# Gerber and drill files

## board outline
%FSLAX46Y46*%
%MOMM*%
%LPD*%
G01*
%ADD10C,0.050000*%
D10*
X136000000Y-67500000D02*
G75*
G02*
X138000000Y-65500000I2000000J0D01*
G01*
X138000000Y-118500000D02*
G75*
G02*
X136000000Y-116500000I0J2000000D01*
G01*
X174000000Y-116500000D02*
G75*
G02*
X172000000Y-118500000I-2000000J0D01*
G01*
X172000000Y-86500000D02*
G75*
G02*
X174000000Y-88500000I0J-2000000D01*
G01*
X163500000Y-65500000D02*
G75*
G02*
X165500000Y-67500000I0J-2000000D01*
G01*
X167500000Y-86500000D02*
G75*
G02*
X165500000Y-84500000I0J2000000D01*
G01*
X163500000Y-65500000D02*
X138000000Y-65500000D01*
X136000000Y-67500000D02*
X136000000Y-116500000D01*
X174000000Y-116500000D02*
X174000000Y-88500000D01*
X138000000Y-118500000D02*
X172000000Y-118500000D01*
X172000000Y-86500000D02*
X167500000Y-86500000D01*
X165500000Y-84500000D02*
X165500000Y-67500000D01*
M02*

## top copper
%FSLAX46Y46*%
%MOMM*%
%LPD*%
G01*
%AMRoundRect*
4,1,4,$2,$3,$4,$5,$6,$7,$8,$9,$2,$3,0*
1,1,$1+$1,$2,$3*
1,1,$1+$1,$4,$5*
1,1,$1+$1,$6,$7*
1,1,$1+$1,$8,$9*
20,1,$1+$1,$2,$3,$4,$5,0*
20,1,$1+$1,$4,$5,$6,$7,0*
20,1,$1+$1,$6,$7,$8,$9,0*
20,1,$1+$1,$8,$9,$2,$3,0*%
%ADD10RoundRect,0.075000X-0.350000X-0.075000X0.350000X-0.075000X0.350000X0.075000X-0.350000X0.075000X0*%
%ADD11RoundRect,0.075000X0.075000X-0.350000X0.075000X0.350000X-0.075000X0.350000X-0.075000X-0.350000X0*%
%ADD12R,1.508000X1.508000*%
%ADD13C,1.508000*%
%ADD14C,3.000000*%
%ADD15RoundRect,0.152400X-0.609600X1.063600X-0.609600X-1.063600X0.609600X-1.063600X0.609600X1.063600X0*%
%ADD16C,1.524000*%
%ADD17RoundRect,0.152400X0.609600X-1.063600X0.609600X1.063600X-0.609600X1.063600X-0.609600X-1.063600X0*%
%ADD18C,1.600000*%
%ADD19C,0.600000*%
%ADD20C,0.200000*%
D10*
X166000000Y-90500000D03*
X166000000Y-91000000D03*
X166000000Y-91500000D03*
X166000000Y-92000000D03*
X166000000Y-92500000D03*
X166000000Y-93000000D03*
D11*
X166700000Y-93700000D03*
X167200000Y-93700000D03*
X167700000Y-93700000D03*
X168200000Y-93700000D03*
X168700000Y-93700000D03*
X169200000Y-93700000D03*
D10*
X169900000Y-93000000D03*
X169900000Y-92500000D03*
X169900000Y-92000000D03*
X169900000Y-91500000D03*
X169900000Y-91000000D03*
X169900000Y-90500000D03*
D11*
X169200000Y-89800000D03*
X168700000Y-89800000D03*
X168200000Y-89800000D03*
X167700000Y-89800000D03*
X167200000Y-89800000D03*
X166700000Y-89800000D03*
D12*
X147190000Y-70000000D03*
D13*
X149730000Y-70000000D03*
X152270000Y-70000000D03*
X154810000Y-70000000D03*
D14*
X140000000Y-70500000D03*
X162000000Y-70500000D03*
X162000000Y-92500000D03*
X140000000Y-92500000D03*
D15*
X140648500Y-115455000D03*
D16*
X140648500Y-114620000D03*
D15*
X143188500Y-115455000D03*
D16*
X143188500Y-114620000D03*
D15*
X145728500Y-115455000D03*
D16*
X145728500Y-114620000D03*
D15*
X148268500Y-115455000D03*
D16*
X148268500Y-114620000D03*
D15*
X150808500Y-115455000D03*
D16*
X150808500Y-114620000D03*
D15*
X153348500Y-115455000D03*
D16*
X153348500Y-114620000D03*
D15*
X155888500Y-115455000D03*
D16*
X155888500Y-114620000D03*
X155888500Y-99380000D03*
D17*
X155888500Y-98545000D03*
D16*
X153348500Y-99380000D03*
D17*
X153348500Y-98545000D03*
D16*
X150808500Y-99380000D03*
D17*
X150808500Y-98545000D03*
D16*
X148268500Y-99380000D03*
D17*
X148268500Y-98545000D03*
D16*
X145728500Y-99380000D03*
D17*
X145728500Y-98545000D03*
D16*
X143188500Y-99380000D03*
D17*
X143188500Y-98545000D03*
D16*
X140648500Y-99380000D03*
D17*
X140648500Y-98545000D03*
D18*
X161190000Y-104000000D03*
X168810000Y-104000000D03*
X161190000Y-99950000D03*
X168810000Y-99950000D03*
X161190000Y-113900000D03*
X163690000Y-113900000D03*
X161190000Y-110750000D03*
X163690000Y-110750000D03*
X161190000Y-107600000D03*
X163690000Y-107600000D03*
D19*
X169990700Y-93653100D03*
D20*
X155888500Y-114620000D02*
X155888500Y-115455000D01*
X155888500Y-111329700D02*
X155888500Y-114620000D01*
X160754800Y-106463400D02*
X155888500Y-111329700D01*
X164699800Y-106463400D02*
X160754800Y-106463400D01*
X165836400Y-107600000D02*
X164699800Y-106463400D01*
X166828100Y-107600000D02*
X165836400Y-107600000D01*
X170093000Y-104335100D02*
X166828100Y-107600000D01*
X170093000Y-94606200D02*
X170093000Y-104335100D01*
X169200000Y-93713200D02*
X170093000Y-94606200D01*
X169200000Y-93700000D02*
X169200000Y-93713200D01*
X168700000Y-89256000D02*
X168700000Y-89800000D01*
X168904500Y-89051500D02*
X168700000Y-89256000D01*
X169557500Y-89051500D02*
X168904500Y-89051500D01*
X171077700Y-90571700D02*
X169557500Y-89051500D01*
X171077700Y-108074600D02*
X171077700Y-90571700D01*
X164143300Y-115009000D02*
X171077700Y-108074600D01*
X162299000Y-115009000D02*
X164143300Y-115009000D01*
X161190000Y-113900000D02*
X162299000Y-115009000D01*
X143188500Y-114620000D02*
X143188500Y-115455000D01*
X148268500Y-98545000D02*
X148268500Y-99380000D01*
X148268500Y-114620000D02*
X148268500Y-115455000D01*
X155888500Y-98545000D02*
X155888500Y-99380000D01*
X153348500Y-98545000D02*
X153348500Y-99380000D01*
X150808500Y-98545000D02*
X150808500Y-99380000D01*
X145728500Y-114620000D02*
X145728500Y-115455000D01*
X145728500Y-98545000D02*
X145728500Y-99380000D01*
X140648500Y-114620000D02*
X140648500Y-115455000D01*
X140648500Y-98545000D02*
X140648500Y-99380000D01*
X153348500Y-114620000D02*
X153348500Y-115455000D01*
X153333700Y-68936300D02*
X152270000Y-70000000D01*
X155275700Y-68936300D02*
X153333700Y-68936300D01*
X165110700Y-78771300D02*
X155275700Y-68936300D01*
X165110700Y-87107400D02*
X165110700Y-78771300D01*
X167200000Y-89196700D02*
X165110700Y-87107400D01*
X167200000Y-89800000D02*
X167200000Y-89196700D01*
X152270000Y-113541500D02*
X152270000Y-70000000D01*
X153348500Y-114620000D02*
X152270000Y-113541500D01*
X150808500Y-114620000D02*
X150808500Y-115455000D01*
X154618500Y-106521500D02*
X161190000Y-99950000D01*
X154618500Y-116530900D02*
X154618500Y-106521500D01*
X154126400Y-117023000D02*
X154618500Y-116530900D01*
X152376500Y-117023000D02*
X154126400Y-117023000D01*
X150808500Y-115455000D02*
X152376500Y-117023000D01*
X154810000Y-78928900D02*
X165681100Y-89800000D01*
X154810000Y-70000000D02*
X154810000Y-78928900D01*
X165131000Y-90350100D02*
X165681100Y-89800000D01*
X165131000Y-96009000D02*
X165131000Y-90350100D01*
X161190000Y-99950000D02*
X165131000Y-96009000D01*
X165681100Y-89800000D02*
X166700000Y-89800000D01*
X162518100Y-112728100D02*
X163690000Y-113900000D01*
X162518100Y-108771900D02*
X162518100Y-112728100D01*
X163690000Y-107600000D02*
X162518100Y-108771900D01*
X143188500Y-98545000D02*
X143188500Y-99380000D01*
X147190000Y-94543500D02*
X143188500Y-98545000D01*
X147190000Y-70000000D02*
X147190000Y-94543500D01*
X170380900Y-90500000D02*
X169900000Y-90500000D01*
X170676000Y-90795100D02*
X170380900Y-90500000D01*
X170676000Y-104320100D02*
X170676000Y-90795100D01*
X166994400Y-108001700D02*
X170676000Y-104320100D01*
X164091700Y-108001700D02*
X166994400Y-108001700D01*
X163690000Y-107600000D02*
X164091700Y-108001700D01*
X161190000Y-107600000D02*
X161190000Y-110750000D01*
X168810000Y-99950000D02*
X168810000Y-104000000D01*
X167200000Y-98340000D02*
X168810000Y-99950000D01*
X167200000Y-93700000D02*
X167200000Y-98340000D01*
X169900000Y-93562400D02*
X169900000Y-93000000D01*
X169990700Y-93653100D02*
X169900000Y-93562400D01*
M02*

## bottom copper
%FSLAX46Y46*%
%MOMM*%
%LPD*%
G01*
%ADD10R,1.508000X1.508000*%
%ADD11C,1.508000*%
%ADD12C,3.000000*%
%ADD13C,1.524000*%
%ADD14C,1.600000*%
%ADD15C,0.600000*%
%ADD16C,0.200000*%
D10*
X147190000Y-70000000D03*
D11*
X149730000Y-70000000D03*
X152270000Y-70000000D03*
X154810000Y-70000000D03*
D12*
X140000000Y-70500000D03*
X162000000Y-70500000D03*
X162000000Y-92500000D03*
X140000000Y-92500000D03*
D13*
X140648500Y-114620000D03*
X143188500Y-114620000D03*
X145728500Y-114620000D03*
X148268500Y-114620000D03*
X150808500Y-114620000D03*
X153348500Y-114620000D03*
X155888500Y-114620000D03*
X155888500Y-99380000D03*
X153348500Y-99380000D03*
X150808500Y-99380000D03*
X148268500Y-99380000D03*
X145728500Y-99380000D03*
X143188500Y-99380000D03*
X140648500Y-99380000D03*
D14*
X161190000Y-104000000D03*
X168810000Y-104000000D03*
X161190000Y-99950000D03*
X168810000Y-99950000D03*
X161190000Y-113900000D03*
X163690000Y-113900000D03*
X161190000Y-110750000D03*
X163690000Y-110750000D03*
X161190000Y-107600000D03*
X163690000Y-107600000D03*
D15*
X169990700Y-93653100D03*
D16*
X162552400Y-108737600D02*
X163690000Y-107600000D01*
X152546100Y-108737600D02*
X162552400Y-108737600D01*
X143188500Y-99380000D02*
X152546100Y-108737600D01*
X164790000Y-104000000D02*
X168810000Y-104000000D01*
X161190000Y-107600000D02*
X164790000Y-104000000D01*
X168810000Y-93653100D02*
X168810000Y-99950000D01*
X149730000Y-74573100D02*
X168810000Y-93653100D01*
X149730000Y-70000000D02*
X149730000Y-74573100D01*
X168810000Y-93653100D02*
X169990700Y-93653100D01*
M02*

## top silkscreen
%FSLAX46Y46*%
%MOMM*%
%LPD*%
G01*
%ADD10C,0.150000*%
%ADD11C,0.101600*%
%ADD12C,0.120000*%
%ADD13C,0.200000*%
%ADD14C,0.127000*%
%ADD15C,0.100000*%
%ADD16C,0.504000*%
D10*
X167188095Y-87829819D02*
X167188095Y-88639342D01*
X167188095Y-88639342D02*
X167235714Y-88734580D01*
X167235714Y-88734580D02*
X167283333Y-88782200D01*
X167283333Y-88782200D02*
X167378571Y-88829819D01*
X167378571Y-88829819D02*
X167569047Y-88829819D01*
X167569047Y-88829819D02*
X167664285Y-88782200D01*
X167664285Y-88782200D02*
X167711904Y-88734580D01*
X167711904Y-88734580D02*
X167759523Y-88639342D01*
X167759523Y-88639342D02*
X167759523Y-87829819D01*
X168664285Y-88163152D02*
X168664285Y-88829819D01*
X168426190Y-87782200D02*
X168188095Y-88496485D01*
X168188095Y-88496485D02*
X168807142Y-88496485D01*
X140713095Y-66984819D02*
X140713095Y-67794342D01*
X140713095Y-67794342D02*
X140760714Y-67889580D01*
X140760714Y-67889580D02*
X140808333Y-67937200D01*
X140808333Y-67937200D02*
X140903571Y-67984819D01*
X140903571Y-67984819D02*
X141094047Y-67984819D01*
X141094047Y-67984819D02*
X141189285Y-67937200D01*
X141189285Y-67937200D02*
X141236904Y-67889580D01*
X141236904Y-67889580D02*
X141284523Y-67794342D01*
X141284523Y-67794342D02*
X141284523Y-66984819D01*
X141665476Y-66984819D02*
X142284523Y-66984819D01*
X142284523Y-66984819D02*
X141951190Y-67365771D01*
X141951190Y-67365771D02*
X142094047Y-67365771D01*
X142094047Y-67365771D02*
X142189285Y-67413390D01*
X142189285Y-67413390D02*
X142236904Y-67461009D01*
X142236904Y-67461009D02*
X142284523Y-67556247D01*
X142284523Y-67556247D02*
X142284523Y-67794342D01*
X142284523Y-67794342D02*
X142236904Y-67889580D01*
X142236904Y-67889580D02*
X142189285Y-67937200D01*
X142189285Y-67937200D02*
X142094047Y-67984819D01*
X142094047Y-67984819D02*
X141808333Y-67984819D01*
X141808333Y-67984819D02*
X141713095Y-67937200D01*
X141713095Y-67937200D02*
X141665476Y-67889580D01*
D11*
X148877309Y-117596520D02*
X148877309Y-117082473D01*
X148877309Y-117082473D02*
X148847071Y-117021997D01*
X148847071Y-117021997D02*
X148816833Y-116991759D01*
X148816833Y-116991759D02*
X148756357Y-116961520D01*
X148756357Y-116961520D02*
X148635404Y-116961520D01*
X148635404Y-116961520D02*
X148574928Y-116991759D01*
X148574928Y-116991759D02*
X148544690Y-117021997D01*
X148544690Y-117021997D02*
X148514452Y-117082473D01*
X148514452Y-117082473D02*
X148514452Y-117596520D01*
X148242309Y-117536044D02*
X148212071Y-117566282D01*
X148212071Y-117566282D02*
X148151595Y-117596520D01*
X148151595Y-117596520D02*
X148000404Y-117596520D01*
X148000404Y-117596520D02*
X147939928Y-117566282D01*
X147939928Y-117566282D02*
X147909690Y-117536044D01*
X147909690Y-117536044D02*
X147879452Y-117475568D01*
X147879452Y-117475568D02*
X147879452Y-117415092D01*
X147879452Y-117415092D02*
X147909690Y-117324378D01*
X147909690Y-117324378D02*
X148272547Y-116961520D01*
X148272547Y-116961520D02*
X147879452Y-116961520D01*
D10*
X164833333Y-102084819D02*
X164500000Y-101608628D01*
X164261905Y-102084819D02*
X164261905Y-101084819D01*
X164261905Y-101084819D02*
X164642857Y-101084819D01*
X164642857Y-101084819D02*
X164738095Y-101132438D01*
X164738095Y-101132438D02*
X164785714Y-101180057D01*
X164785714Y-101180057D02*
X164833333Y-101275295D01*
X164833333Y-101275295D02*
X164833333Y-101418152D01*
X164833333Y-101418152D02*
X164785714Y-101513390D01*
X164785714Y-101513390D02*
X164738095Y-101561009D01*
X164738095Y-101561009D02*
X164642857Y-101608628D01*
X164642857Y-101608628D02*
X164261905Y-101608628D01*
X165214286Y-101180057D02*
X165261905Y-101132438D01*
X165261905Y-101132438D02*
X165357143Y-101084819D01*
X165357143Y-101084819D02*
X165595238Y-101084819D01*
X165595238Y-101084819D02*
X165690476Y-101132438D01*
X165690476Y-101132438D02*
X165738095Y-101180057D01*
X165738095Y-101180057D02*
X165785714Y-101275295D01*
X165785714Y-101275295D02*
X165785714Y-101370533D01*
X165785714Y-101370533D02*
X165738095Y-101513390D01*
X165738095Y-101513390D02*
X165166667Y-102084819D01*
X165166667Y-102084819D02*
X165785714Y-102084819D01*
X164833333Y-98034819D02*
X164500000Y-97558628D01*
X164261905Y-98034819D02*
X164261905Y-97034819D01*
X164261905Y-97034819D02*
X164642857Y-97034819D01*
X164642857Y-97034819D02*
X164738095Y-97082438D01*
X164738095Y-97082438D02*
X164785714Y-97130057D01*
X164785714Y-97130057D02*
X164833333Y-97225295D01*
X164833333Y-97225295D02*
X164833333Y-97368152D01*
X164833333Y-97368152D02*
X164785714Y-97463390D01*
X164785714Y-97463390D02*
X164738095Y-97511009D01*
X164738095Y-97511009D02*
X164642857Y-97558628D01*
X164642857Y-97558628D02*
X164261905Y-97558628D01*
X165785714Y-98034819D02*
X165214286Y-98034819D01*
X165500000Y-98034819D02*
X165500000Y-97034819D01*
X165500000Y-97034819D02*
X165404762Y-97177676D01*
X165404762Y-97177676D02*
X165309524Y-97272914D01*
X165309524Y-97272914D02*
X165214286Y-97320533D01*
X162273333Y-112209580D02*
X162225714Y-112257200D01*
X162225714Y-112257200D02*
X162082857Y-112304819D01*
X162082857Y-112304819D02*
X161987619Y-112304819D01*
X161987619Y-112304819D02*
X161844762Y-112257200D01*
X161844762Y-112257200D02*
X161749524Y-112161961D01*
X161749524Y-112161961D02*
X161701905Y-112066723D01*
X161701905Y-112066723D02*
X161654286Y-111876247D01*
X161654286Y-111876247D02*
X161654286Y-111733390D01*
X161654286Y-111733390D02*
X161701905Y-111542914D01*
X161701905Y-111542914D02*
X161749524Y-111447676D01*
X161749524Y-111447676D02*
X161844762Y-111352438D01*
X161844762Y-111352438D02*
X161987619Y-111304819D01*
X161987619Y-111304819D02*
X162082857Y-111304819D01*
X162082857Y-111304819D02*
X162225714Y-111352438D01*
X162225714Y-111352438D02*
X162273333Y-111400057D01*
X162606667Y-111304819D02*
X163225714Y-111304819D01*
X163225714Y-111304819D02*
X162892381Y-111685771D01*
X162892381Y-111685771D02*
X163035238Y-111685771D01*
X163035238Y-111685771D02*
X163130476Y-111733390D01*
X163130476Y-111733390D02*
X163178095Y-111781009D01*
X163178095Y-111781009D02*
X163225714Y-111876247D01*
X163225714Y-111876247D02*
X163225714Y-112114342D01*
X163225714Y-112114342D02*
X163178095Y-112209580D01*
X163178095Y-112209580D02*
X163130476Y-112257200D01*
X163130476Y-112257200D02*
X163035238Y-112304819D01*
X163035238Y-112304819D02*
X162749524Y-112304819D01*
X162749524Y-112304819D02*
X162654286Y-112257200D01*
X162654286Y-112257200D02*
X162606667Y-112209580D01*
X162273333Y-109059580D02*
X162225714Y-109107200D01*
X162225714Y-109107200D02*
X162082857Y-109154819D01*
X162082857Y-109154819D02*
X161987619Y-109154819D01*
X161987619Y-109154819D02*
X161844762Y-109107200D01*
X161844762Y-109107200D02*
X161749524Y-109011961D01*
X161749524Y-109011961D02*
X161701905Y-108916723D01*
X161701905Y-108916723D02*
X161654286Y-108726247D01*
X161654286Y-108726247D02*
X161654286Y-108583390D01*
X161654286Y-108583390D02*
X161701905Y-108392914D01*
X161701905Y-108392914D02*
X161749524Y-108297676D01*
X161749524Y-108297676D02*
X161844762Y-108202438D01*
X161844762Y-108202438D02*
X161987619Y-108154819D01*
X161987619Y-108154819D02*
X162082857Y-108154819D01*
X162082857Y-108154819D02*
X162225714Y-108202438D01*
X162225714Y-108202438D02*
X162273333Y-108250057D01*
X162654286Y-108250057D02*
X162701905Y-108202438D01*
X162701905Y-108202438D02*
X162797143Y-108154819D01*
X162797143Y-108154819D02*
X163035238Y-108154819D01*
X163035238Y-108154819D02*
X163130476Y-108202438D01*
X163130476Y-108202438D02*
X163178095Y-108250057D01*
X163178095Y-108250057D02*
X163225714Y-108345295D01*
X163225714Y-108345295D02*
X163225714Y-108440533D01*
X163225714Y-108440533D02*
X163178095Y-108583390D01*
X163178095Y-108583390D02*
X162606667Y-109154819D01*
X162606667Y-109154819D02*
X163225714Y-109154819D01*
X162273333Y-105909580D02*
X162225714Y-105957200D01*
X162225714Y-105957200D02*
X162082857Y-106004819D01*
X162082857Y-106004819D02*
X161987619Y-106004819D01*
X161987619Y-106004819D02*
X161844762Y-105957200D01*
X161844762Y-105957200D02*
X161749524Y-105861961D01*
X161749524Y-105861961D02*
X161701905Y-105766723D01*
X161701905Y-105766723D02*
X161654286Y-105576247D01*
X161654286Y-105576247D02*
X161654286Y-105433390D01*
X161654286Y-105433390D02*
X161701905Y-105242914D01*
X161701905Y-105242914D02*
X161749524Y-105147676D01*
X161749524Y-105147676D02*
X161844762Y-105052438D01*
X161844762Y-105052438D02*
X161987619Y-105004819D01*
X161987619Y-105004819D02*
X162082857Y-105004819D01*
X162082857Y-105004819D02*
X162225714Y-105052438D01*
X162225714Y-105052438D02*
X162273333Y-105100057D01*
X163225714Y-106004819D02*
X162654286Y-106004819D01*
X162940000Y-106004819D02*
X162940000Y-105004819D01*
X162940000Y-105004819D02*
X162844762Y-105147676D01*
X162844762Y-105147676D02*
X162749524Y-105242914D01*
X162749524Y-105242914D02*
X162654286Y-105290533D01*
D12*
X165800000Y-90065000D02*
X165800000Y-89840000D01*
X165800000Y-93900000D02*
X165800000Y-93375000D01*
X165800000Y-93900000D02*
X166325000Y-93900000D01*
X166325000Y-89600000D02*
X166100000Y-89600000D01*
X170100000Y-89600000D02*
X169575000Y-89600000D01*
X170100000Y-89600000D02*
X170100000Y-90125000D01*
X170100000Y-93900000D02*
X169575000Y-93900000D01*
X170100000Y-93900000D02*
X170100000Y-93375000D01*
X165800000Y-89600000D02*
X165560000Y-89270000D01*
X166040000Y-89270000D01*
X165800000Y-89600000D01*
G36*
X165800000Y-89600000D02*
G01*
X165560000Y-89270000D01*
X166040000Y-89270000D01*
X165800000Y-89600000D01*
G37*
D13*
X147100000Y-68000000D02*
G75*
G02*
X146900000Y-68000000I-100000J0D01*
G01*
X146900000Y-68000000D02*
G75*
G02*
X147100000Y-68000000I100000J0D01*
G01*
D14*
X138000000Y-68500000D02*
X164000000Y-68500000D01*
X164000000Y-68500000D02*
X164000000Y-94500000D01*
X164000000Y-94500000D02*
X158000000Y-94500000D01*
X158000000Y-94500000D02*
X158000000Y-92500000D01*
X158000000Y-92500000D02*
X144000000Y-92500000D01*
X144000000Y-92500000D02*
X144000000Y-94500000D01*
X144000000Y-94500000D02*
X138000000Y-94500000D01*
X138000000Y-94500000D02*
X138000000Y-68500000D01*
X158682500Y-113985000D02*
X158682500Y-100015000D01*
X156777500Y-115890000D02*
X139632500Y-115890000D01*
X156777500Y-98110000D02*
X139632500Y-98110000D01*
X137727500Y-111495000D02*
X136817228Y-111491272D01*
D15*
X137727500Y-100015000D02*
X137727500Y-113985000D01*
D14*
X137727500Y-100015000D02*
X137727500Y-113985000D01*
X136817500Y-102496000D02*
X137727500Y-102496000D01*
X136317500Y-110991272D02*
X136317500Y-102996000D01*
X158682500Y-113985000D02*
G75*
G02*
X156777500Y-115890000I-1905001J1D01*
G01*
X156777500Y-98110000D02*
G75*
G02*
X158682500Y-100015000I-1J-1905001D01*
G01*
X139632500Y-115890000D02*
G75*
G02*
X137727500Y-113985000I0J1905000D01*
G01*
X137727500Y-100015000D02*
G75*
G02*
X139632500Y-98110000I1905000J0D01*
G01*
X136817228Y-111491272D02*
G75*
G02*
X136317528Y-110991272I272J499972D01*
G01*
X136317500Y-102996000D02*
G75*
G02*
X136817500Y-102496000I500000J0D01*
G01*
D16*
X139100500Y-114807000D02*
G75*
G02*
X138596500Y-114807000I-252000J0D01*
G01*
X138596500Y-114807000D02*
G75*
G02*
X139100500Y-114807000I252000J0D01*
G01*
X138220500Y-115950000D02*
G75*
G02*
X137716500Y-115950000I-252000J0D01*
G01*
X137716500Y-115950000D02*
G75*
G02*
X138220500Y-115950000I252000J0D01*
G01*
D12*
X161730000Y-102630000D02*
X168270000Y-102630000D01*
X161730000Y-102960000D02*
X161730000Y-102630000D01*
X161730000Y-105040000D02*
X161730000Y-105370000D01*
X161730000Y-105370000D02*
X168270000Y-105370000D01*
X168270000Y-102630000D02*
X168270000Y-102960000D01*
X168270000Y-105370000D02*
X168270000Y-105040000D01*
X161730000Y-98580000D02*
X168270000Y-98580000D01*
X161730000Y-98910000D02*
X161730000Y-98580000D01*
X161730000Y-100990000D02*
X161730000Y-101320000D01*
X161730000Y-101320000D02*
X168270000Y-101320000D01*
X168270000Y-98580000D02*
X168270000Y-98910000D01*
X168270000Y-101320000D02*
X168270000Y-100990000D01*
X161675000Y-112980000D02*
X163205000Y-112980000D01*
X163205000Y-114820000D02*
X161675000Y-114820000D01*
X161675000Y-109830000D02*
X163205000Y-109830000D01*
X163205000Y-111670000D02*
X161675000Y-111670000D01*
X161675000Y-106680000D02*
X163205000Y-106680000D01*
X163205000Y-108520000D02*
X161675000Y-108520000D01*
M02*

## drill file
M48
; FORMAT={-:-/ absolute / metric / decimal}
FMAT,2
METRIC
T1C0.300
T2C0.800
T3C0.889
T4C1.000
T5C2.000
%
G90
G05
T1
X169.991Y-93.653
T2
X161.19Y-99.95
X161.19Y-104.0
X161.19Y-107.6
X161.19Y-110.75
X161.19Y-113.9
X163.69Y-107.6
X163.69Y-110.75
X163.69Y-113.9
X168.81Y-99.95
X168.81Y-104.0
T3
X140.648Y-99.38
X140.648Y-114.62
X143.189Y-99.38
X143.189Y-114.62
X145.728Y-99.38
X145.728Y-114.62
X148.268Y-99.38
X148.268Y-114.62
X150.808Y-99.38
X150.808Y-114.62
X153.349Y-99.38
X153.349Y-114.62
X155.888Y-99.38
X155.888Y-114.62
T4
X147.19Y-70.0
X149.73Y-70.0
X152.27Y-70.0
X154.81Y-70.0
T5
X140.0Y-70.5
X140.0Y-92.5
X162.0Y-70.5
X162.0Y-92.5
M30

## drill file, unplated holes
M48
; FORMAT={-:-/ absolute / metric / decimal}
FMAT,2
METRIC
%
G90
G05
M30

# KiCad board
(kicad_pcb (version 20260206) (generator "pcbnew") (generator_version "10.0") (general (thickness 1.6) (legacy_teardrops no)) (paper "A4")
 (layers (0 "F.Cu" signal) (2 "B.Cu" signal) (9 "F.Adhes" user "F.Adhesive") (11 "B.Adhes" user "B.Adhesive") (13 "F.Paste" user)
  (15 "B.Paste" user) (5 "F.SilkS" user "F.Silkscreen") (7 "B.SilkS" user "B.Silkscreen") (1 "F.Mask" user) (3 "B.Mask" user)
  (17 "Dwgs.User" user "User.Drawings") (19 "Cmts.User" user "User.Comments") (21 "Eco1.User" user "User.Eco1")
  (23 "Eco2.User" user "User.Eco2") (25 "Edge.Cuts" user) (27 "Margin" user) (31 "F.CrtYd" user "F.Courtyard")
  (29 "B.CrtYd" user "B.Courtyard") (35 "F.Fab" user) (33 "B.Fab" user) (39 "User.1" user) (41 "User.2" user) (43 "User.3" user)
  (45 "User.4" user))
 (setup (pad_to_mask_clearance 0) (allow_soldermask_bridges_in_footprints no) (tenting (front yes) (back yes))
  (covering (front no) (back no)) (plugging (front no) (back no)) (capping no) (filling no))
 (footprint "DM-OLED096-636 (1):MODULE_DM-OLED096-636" (layer "F.Cu") (at 151 81.5)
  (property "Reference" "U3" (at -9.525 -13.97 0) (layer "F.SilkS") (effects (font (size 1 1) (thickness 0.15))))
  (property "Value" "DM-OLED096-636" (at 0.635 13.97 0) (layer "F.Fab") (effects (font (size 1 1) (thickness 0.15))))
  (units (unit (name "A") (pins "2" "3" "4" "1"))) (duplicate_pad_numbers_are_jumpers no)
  (fp_line (start -13 -13) (end 13 -13) (stroke (width 0.127) (type solid)) (layer "F.SilkS"))
  (fp_line (start -13 13) (end -13 -13) (stroke (width 0.127) (type solid)) (layer "F.SilkS"))
  (fp_line (start -7 11) (end -7 13) (stroke (width 0.127) (type solid)) (layer "F.SilkS"))
  (fp_line (start -7 13) (end -13 13) (stroke (width 0.127) (type solid)) (layer "F.SilkS"))
  (fp_line (start 7 11) (end -7 11) (stroke (width 0.127) (type solid)) (layer "F.SilkS"))
  (fp_line (start 7 13) (end 7 11) (stroke (width 0.127) (type solid)) (layer "F.SilkS"))
  (fp_line (start 13 -13) (end 13 13) (stroke (width 0.127) (type solid)) (layer "F.SilkS"))
  (fp_line (start 13 13) (end 7 13) (stroke (width 0.127) (type solid)) (layer "F.SilkS"))
  (fp_circle (center -4 -13.5) (end -3.9 -13.5) (stroke (width 0.2) (type solid)) (fill no) (layer "F.SilkS"))
  (pad "1" thru_hole rect (at -3.81 -11.5) (size 1.508 1.508) (drill 1) (layers "*.Cu" "*.Mask") (remove_unused_layers no) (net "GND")
   (solder_mask_margin 0.102))
  (pad "2" thru_hole circle (at -1.27 -11.5) (size 1.508 1.508) (drill 1) (layers "*.Cu" "*.Mask") (remove_unused_layers no) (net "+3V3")
   (solder_mask_margin 0.102))
  (pad "3" thru_hole circle (at 1.27 -11.5) (size 1.508 1.508) (drill 1) (layers "*.Cu" "*.Mask") (remove_unused_layers no) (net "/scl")
   (solder_mask_margin 0.102))
  (pad "4" thru_hole circle (at 3.81 -11.5) (size 1.508 1.508) (drill 1) (layers "*.Cu" "*.Mask") (remove_unused_layers no) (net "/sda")
   (solder_mask_margin 0.102))
  (pad "S1" thru_hole circle (at -11 -11) (size 3 3) (drill 2) (layers "*.Cu" "*.Mask") (remove_unused_layers no) (solder_mask_margin 0.102))
  (pad "S2" thru_hole circle (at 11 -11) (size 3 3) (drill 2) (layers "*.Cu" "*.Mask") (remove_unused_layers no) (solder_mask_margin 0.102))
  (pad "S3" thru_hole circle (at 11 11) (size 3 3) (drill 2) (layers "*.Cu" "*.Mask") (remove_unused_layers no) (solder_mask_margin 0.102))
  (pad "S4" thru_hole circle (at -11 11) (size 3 3) (drill 2) (layers "*.Cu" "*.Mask") (remove_unused_layers no) (solder_mask_margin 0.102)))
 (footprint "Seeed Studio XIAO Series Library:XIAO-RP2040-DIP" (layer "F.Cu") (at 148.2685 107 180)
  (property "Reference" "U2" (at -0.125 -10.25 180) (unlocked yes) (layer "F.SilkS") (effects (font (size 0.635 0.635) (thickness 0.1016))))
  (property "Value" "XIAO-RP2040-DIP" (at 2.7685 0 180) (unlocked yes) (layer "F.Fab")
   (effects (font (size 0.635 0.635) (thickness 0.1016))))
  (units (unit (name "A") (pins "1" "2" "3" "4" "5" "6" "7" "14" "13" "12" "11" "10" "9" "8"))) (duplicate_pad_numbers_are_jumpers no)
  (fp_line (start 11.951 -3.991272) (end 11.951 4.004) (stroke (width 0.127) (type solid)) (layer "F.SilkS"))
  (fp_line (start 11.451 4.504) (end 10.541 4.504) (stroke (width 0.127) (type solid)) (layer "F.SilkS"))
  (fp_line (start 10.541 6.985) (end 10.541 -6.985) (stroke (width 0.1) (type solid)) (layer "F.SilkS"))
  (fp_line (start 10.541 6.985) (end 10.541 -6.985) (stroke (width 0.127) (type solid)) (layer "F.SilkS"))
  (fp_line (start 10.541 -4.495) (end 11.451272 -4.491272) (stroke (width 0.127) (type solid)) (layer "F.SilkS"))
  (fp_line (start -8.509 8.89) (end 8.636 8.89) (stroke (width 0.127) (type solid)) (layer "F.SilkS"))
  (fp_line (start -8.509 -8.89) (end 8.636 -8.89) (stroke (width 0.127) (type solid)) (layer "F.SilkS"))
  (fp_line (start -10.414 -6.985) (end -10.414 6.985) (stroke (width 0.127) (type solid)) (layer "F.SilkS"))
  (fp_arc (start 11.951 4.004) (mid 11.804553 4.357553) (end 11.451 4.504) (stroke (width 0.127) (type default)) (layer "F.SilkS"))
  (fp_arc (start 11.451272 -4.491272) (mid 11.804644 -4.344724) (end 11.951 -3.991272) (stroke (width 0.127) (type default))
   (layer "F.SilkS"))
  (fp_arc (start 10.541 6.985) (mid 9.983038 8.332038) (end 8.636 8.89) (stroke (width 0.127) (type solid)) (layer "F.SilkS"))
  (fp_arc (start 8.636 -8.89) (mid 9.983038 -8.332038) (end 10.541 -6.985) (stroke (width 0.127) (type solid)) (layer "F.SilkS"))
  (fp_arc (start -8.509 8.89) (mid -9.856038 8.332038) (end -10.414 6.985) (stroke (width 0.127) (type solid)) (layer "F.SilkS"))
  (fp_arc (start -10.414 -6.985) (mid -9.856038 -8.332038) (end -8.509 -8.89) (stroke (width 0.127) (type solid)) (layer "F.SilkS"))
  (fp_circle (center 10.3 -8.95) (end 10.554 -8.95) (stroke (width 0.5) (type solid)) (fill yes) (layer "F.SilkS"))
  (fp_circle (center 9.42 -7.807) (end 9.674 -7.807) (stroke (width 0.5) (type solid)) (fill yes) (layer "F.SilkS"))
  (pad "1" smd roundrect (at 7.62 -8.455 270) (size 2.432 1.524) (layers "F.Cu" "F.Mask") (roundrect_rratio 0.1)
   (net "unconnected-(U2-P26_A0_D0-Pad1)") (thermal_bridge_angle 45))
  (pad "1" thru_hole circle (at 7.62 -7.62 270) (size 1.524 1.524) (drill 0.889) (layers "*.Cu" "*.Mask") (remove_unused_layers no)
   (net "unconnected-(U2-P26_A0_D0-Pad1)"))
  (pad "2" smd roundrect (at 5.08 -8.455 270) (size 2.432 1.524) (layers "F.Cu" "F.Mask") (roundrect_rratio 0.1)
   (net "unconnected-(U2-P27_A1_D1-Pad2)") (thermal_bridge_angle 45))
  (pad "2" thru_hole circle (at 5.08 -7.62 270) (size 1.524 1.524) (drill 0.889) (layers "*.Cu" "*.Mask") (remove_unused_layers no)
   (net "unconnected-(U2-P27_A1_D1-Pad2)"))
  (pad "3" smd roundrect (at 2.54 -8.455 270) (size 2.432 1.524) (layers "F.Cu" "F.Mask") (roundrect_rratio 0.1)
   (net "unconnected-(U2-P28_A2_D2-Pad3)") (thermal_bridge_angle 45))
  (pad "3" thru_hole circle (at 2.54 -7.62 270) (size 1.524 1.524) (drill 0.889) (layers "*.Cu" "*.Mask") (remove_unused_layers no)
   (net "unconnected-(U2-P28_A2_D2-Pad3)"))
  (pad "4" smd roundrect (at 0 -8.455 270) (size 2.432 1.524) (layers "F.Cu" "F.Mask") (roundrect_rratio 0.1)
   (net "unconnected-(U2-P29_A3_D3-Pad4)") (thermal_bridge_angle 45))
  (pad "4" thru_hole circle (at 0 -7.62 270) (size 1.524 1.524) (drill 0.889) (layers "*.Cu" "*.Mask") (remove_unused_layers no)
   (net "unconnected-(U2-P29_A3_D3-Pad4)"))
  (pad "5" smd roundrect (at -2.54 -8.455 270) (size 2.432 1.524) (layers "F.Cu" "F.Mask") (roundrect_rratio 0.1) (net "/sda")
   (thermal_bridge_angle 45))
  (pad "5" thru_hole circle (at -2.54 -7.62 270) (size 1.524 1.524) (drill 0.889) (layers "*.Cu" "*.Mask") (remove_unused_layers no)
   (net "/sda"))
  (pad "6" smd roundrect (at -5.08 -8.455 270) (size 2.432 1.524) (layers "F.Cu" "F.Mask") (roundrect_rratio 0.1) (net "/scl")
   (thermal_bridge_angle 45))
  (pad "6" thru_hole circle (at -5.08 -7.62 270) (size 1.524 1.524) (drill 0.889) (layers "*.Cu" "*.Mask") (remove_unused_layers no)
   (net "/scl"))
  (pad "7" smd roundrect (at -7.62 -8.455 270) (size 2.432 1.524) (layers "F.Cu" "F.Mask") (roundrect_rratio 0.1) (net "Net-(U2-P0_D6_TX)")
   (thermal_bridge_angle 45))
  (pad "7" thru_hole circle (at -7.62 -7.62 270) (size 1.524 1.524) (drill 0.889) (layers "*.Cu" "*.Mask") (remove_unused_layers no)
   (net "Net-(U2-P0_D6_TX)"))
  (pad "8" thru_hole circle (at -7.62 7.62 90) (size 1.524 1.524) (drill 0.889) (layers "*.Cu" "*.Mask") (remove_unused_layers no)
   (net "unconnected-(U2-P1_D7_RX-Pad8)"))
  (pad "8" smd roundrect (at -7.62 8.455 90) (size 2.432 1.524) (layers "F.Cu" "F.Mask") (roundrect_rratio 0.1)
   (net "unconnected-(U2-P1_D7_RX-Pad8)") (thermal_bridge_angle 45))
  (pad "9" thru_hole circle (at -5.08 7.62 90) (size 1.524 1.524) (drill 0.889) (layers "*.Cu" "*.Mask") (remove_unused_layers no)
   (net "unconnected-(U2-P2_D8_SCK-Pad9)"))
  (pad "9" smd roundrect (at -5.08 8.455 90) (size 2.432 1.524) (layers "F.Cu" "F.Mask") (roundrect_rratio 0.1)
   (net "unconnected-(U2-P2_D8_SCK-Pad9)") (thermal_bridge_angle 45))
  (pad "10" thru_hole circle (at -2.54 7.62 90) (size 1.524 1.524) (drill 0.889) (layers "*.Cu" "*.Mask") (remove_unused_layers no)
   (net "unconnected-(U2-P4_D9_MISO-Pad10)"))
  (pad "10" smd roundrect (at -2.54 8.455 90) (size 2.432 1.524) (layers "F.Cu" "F.Mask") (roundrect_rratio 0.1)
   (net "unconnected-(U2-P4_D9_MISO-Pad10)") (thermal_bridge_angle 45))
  (pad "11" thru_hole circle (at 0 7.62 90) (size 1.524 1.524) (drill 0.889) (layers "*.Cu" "*.Mask") (remove_unused_layers no)
   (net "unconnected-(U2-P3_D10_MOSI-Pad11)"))
  (pad "11" smd roundrect (at 0 8.455 90) (size 2.432 1.524) (layers "F.Cu" "F.Mask") (roundrect_rratio 0.1)
   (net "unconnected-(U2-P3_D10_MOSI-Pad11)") (thermal_bridge_angle 45))
  (pad "12" thru_hole circle (at 2.54 7.62 90) (size 1.524 1.524) (drill 0.889) (layers "*.Cu" "*.Mask") (remove_unused_layers no)
   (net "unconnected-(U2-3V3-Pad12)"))
  (pad "12" smd roundrect (at 2.54 8.455 90) (size 2.432 1.524) (layers "F.Cu" "F.Mask") (roundrect_rratio 0.1)
   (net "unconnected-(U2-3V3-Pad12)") (thermal_bridge_angle 45))
  (pad "13" thru_hole circle (at 5.08 7.62 90) (size 1.524 1.524) (drill 0.889) (layers "*.Cu" "*.Mask") (remove_unused_layers no)
   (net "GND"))
  (pad "13" smd roundrect (at 5.08 8.455 90) (size 2.432 1.524) (layers "F.Cu" "F.Mask") (roundrect_rratio 0.1) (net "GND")
   (thermal_bridge_angle 45))
  (pad "14" thru_hole circle (at 7.62 7.62 90) (size 1.524 1.524) (drill 0.889) (layers "*.Cu" "*.Mask") (remove_unused_layers no)
   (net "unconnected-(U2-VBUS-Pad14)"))
  (pad "14" smd roundrect (at 7.62 8.455 90) (size 2.432 1.524) (layers "F.Cu" "F.Mask") (roundrect_rratio 0.1)
   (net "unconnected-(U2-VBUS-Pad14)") (thermal_bridge_angle 45)))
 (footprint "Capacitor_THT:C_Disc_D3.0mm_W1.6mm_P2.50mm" (layer "F.Cu") (at 161.19 110.75)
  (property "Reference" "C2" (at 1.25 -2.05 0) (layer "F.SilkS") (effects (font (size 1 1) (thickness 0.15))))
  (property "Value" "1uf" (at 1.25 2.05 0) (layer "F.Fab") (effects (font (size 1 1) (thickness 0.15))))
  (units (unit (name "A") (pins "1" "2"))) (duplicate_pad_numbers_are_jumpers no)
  (fp_line (start 0.485 -0.92) (end 2.015 -0.92) (stroke (width 0.12) (type solid)) (layer "F.SilkS"))
  (fp_line (start 2.015 0.92) (end 0.485 0.92) (stroke (width 0.12) (type solid)) (layer "F.SilkS"))
  (pad "1" thru_hole circle (at 0 0) (size 1.6 1.6) (drill 0.8) (layers "*.Cu" "*.Mask") (remove_unused_layers no) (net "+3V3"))
  (pad "2" thru_hole circle (at 2.5 0) (size 1.6 1.6) (drill 0.8) (layers "*.Cu" "*.Mask") (remove_unused_layers no)
   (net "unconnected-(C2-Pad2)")))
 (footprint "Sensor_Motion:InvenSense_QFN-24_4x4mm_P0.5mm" (layer "F.Cu") (at 167.95 91.75)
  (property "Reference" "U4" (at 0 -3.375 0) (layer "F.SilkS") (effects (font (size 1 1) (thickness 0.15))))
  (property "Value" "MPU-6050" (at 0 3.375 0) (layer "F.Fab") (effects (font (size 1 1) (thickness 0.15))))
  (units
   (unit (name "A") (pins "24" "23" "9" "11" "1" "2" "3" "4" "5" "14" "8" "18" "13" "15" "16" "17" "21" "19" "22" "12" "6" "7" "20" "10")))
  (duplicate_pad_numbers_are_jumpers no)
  (fp_line (start -2.15 -1.685) (end -2.15 -1.91) (stroke (width 0.12) (type solid)) (layer "F.SilkS"))
  (fp_line (start -2.15 2.15) (end -2.15 1.625) (stroke (width 0.12) (type solid)) (layer "F.SilkS"))
  (fp_line (start -2.15 2.15) (end -1.625 2.15) (stroke (width 0.12) (type solid)) (layer "F.SilkS"))
  (fp_line (start -1.625 -2.15) (end -1.85 -2.15) (stroke (width 0.12) (type solid)) (layer "F.SilkS"))
  (fp_line (start 2.15 -2.15) (end 1.625 -2.15) (stroke (width 0.12) (type solid)) (layer "F.SilkS"))
  (fp_line (start 2.15 -2.15) (end 2.15 -1.625) (stroke (width 0.12) (type solid)) (layer "F.SilkS"))
  (fp_line (start 2.15 2.15) (end 1.625 2.15) (stroke (width 0.12) (type solid)) (layer "F.SilkS"))
  (fp_line (start 2.15 2.15) (end 2.15 1.625) (stroke (width 0.12) (type solid)) (layer "F.SilkS"))
  (fp_poly
   (pts (xy -2.15 -2.15) (xy -2.39 -2.48) (xy -1.91 -2.48) (xy -2.15 -2.15)) (stroke (width 0.12) (type solid)) (fill yes) (layer "F.SilkS"))
  (pad "1" smd roundrect (at -1.95 -1.25) (size 0.85 0.3) (layers "F.Cu" "F.Mask" "F.Paste") (roundrect_rratio 0.25)
   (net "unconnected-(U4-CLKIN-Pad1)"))
  (pad "2" smd roundrect (at -1.95 -0.75) (size 0.85 0.3) (layers "F.Cu" "F.Mask" "F.Paste") (roundrect_rratio 0.25)
   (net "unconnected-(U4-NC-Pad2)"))
  (pad "3" smd roundrect (at -1.95 -0.25) (size 0.85 0.3) (layers "F.Cu" "F.Mask" "F.Paste") (roundrect_rratio 0.25)
   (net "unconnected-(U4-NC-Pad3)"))
  (pad "4" smd roundrect (at -1.95 0.25) (size 0.85 0.3) (layers "F.Cu" "F.Mask" "F.Paste") (roundrect_rratio 0.25)
   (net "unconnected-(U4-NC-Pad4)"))
  (pad "5" smd roundrect (at -1.95 0.75) (size 0.85 0.3) (layers "F.Cu" "F.Mask" "F.Paste") (roundrect_rratio 0.25)
   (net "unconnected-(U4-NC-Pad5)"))
  (pad "6" smd roundrect (at -1.95 1.25) (size 0.85 0.3) (layers "F.Cu" "F.Mask" "F.Paste") (roundrect_rratio 0.25)
   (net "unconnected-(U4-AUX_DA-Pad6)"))
  (pad "7" smd roundrect (at -1.25 1.95 90) (size 0.85 0.3) (layers "F.Cu" "F.Mask" "F.Paste") (roundrect_rratio 0.25)
   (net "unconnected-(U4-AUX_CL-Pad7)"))
  (pad "8" smd roundrect (at -0.75 1.95 90) (size 0.85 0.3) (layers "F.Cu" "F.Mask" "F.Paste") (roundrect_rratio 0.25) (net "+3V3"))
  (pad "9" smd roundrect (at -0.25 1.95 90) (size 0.85 0.3) (layers "F.Cu" "F.Mask" "F.Paste") (roundrect_rratio 0.25)
   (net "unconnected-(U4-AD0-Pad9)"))
  (pad "10" smd roundrect (at 0.25 1.95 90) (size 0.85 0.3) (layers "F.Cu" "F.Mask" "F.Paste") (roundrect_rratio 0.25)
   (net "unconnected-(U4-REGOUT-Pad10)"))
  (pad "11" smd roundrect (at 0.75 1.95 90) (size 0.85 0.3) (layers "F.Cu" "F.Mask" "F.Paste") (roundrect_rratio 0.25)
   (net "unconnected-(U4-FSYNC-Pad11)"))
  (pad "12" smd roundrect (at 1.25 1.95 90) (size 0.85 0.3) (layers "F.Cu" "F.Mask" "F.Paste") (roundrect_rratio 0.25)
   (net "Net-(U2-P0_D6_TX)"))
  (pad "13" smd roundrect (at 1.95 1.25) (size 0.85 0.3) (layers "F.Cu" "F.Mask" "F.Paste") (roundrect_rratio 0.25) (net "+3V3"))
  (pad "14" smd roundrect (at 1.95 0.75) (size 0.85 0.3) (layers "F.Cu" "F.Mask" "F.Paste") (roundrect_rratio 0.25)
   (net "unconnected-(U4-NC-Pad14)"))
  (pad "15" smd roundrect (at 1.95 0.25) (size 0.85 0.3) (layers "F.Cu" "F.Mask" "F.Paste") (roundrect_rratio 0.25)
   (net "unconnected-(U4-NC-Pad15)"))
  (pad "16" smd roundrect (at 1.95 -0.25) (size 0.85 0.3) (layers "F.Cu" "F.Mask" "F.Paste") (roundrect_rratio 0.25)
   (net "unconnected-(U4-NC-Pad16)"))
  (pad "17" smd roundrect (at 1.95 -0.75) (size 0.85 0.3) (layers "F.Cu" "F.Mask" "F.Paste") (roundrect_rratio 0.25)
   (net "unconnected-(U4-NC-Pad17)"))
  (pad "18" smd roundrect (at 1.95 -1.25) (size 0.85 0.3) (layers "F.Cu" "F.Mask" "F.Paste") (roundrect_rratio 0.25) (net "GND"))
  (pad "19" smd roundrect (at 1.25 -1.95 90) (size 0.85 0.3) (layers "F.Cu" "F.Mask" "F.Paste") (roundrect_rratio 0.25)
   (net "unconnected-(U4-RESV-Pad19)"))
  (pad "20" smd roundrect (at 0.75 -1.95 90) (size 0.85 0.3) (layers "F.Cu" "F.Mask" "F.Paste") (roundrect_rratio 0.25)
   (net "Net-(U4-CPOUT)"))
  (pad "21" smd roundrect (at 0.25 -1.95 90) (size 0.85 0.3) (layers "F.Cu" "F.Mask" "F.Paste") (roundrect_rratio 0.25)
   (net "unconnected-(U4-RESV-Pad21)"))
  (pad "22" smd roundrect (at -0.25 -1.95 90) (size 0.85 0.3) (layers "F.Cu" "F.Mask" "F.Paste") (roundrect_rratio 0.25)
   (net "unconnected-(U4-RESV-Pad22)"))
  (pad "23" smd roundrect (at -0.75 -1.95 90) (size 0.85 0.3) (layers "F.Cu" "F.Mask" "F.Paste") (roundrect_rratio 0.25) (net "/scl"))
  (pad "24" smd roundrect (at -1.25 -1.95 90) (size 0.85 0.3) (layers "F.Cu" "F.Mask" "F.Paste") (roundrect_rratio 0.25) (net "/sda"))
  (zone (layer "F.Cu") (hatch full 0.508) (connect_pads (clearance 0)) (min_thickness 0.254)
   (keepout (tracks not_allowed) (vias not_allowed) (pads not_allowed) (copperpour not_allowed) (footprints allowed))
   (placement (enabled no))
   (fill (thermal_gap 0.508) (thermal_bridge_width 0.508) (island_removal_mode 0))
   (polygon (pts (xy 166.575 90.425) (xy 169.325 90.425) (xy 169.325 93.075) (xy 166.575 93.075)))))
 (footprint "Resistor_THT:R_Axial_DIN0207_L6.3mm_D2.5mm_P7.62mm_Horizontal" (layer "F.Cu") (at 161.19 104)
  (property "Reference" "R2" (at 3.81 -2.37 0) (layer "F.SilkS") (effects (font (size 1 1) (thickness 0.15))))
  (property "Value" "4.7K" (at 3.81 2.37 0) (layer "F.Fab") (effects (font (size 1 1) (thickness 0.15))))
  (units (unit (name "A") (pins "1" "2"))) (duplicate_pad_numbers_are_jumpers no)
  (fp_line (start 0.54 -1.37) (end 7.08 -1.37) (stroke (width 0.12) (type solid)) (layer "F.SilkS"))
  (fp_line (start 0.54 -1.04) (end 0.54 -1.37) (stroke (width 0.12) (type solid)) (layer "F.SilkS"))
  (fp_line (start 0.54 1.04) (end 0.54 1.37) (stroke (width 0.12) (type solid)) (layer "F.SilkS"))
  (fp_line (start 0.54 1.37) (end 7.08 1.37) (stroke (width 0.12) (type solid)) (layer "F.SilkS"))
  (fp_line (start 7.08 -1.37) (end 7.08 -1.04) (stroke (width 0.12) (type solid)) (layer "F.SilkS"))
  (fp_line (start 7.08 1.37) (end 7.08 1.04) (stroke (width 0.12) (type solid)) (layer "F.SilkS"))
  (pad "1" thru_hole circle (at 0 0) (size 1.6 1.6) (drill 0.8) (layers "*.Cu" "*.Mask") (remove_unused_layers no) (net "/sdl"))
  (pad "2" thru_hole circle (at 7.62 0) (size 1.6 1.6) (drill 0.8) (layers "*.Cu" "*.Mask") (remove_unused_layers no) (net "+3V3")))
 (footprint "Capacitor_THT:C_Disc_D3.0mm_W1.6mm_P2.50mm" (layer "F.Cu") (at 161.19 107.6)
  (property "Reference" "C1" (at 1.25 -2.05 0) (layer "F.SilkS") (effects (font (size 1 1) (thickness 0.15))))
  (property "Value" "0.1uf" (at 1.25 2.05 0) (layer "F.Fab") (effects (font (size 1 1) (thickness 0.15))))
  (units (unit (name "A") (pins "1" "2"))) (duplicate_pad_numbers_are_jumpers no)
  (fp_line (start 0.485 -0.92) (end 2.015 -0.92) (stroke (width 0.12) (type solid)) (layer "F.SilkS"))
  (fp_line (start 2.015 0.92) (end 0.485 0.92) (stroke (width 0.12) (type solid)) (layer "F.SilkS"))
  (pad "1" thru_hole circle (at 0 0) (size 1.6 1.6) (drill 0.8) (layers "*.Cu" "*.Mask") (remove_unused_layers no) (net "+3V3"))
  (pad "2" thru_hole circle (at 2.5 0) (size 1.6 1.6) (drill 0.8) (layers "*.Cu" "*.Mask") (remove_unused_layers no) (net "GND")))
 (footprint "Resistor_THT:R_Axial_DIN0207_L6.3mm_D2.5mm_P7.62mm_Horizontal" (layer "F.Cu") (at 161.19 99.95)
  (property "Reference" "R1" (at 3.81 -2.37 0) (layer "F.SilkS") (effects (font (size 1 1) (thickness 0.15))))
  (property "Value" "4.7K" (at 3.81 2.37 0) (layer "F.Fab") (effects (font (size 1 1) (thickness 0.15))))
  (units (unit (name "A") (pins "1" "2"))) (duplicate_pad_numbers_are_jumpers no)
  (fp_line (start 0.54 -1.37) (end 7.08 -1.37) (stroke (width 0.12) (type solid)) (layer "F.SilkS"))
  (fp_line (start 0.54 -1.04) (end 0.54 -1.37) (stroke (width 0.12) (type solid)) (layer "F.SilkS"))
  (fp_line (start 0.54 1.04) (end 0.54 1.37) (stroke (width 0.12) (type solid)) (layer "F.SilkS"))
  (fp_line (start 0.54 1.37) (end 7.08 1.37) (stroke (width 0.12) (type solid)) (layer "F.SilkS"))
  (fp_line (start 7.08 -1.37) (end 7.08 -1.04) (stroke (width 0.12) (type solid)) (layer "F.SilkS"))
  (fp_line (start 7.08 1.37) (end 7.08 1.04) (stroke (width 0.12) (type solid)) (layer "F.SilkS"))
  (pad "1" thru_hole circle (at 0 0) (size 1.6 1.6) (drill 0.8) (layers "*.Cu" "*.Mask") (remove_unused_layers no) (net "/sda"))
  (pad "2" thru_hole circle (at 7.62 0) (size 1.6 1.6) (drill 0.8) (layers "*.Cu" "*.Mask") (remove_unused_layers no) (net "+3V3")))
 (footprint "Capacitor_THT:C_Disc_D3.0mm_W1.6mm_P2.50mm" (layer "F.Cu") (at 161.19 113.9)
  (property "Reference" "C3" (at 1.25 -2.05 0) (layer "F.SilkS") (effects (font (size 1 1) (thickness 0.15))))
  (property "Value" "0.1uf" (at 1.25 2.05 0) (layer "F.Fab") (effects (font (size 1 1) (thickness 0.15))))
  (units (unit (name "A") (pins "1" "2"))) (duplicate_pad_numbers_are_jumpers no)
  (fp_line (start 0.485 -0.92) (end 2.015 -0.92) (stroke (width 0.12) (type solid)) (layer "F.SilkS"))
  (fp_line (start 2.015 0.92) (end 0.485 0.92) (stroke (width 0.12) (type solid)) (layer "F.SilkS"))
  (pad "1" thru_hole circle (at 0 0) (size 1.6 1.6) (drill 0.8) (layers "*.Cu" "*.Mask") (remove_unused_layers no) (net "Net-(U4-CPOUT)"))
  (pad "2" thru_hole circle (at 2.5 0) (size 1.6 1.6) (drill 0.8) (layers "*.Cu" "*.Mask") (remove_unused_layers no) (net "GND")))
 (gr_line (start 136 67.5) (end 136 116.5) (stroke (width 0.05) (type default)) (layer "Edge.Cuts"))
 (gr_arc (start 136 67.5) (mid 136.585786 66.085786) (end 138 65.5) (stroke (width 0.05) (type default)) (layer "Edge.Cuts"))
 (gr_arc (start 138 118.5) (mid 136.585786 117.914214) (end 136 116.5) (stroke (width 0.05) (type default)) (layer "Edge.Cuts"))
 (gr_line (start 138 118.5) (end 172 118.5) (stroke (width 0.05) (type default)) (layer "Edge.Cuts"))
 (gr_line (start 163.5 65.5) (end 138 65.5) (stroke (width 0.05) (type default)) (layer "Edge.Cuts"))
 (gr_arc (start 163.5 65.5) (mid 164.914214 66.085786) (end 165.5 67.5) (stroke (width 0.05) (type default)) (layer "Edge.Cuts"))
 (gr_line (start 165.5 84.5) (end 165.5 67.5) (stroke (width 0.05) (type default)) (layer "Edge.Cuts"))
 (gr_arc (start 167.5 86.5) (mid 166.085786 85.914214) (end 165.5 84.5) (stroke (width 0.05) (type default)) (layer "Edge.Cuts"))
 (gr_line (start 172 86.5) (end 167.5 86.5) (stroke (width 0.05) (type default)) (layer "Edge.Cuts"))
 (gr_arc (start 172 86.5) (mid 173.414214 87.085786) (end 174 88.5) (stroke (width 0.05) (type default)) (layer "Edge.Cuts"))
 (gr_arc (start 174 116.5) (mid 173.414214 117.914214) (end 172 118.5) (stroke (width 0.05) (type default)) (layer "Edge.Cuts"))
 (gr_line (start 174 116.5) (end 174 88.5) (stroke (width 0.05) (type default)) (layer "Edge.Cuts"))
 (segment (start 161.19 107.6) (end 161.19 110.75) (width 0.2) (layer "F.Cu") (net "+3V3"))
 (segment (start 169.9907 93.6531) (end 169.9 93.5624) (width 0.2) (layer "F.Cu") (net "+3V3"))
 (segment (start 167.2 98.34) (end 168.81 99.95) (width 0.2) (layer "F.Cu") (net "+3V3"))
 (segment (start 167.2 93.7) (end 167.2 98.34) (width 0.2) (layer "F.Cu") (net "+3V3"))
 (segment (start 169.9 93.5624) (end 169.9 93) (width 0.2) (layer "F.Cu") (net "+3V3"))
 (segment (start 168.81 99.95) (end 168.81 104) (width 0.2) (layer "F.Cu") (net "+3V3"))
 (via (at 169.9907 93.6531) (size 0.6) (drill 0.3) (layers "F.Cu" "B.Cu") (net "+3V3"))
 (segment (start 168.81 93.6531) (end 168.81 99.95) (width 0.2) (layer "B.Cu") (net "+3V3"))
 (segment (start 164.79 104) (end 168.81 104) (width 0.2) (layer "B.Cu") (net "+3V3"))
 (segment (start 161.19 107.6) (end 164.79 104) (width 0.2) (layer "B.Cu") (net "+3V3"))
 (segment (start 149.73 70) (end 149.73 74.5731) (width 0.2) (layer "B.Cu") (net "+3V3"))
 (segment (start 168.81 93.6531) (end 169.9907 93.6531) (width 0.2) (layer "B.Cu") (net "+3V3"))
 (segment (start 149.73 74.5731) (end 168.81 93.6531) (width 0.2) (layer "B.Cu") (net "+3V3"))
 (segment (start 166.9944 108.0017) (end 170.676 104.3201) (width 0.2) (layer "F.Cu") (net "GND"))
 (segment (start 163.69 107.6) (end 164.0917 108.0017) (width 0.2) (layer "F.Cu") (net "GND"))
 (segment (start 170.676 90.7951) (end 170.3809 90.5) (width 0.2) (layer "F.Cu") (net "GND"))
 (segment (start 170.3809 90.5) (end 169.9 90.5) (width 0.2) (layer "F.Cu") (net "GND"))
 (segment (start 147.19 94.5435) (end 143.1885 98.545) (width 0.2) (layer "F.Cu") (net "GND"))
 (segment (start 163.69 107.6) (end 162.5181 108.7719) (width 0.2) (layer "F.Cu") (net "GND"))
 (segment (start 147.19 70) (end 147.19 94.5435) (width 0.2) (layer "F.Cu") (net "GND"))
 (segment (start 143.1885 98.545) (end 143.1885 99.38) (width 0.2) (layer "F.Cu") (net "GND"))
 (segment (start 170.676 104.3201) (end 170.676 90.7951) (width 0.2) (layer "F.Cu") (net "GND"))
 (segment (start 164.0917 108.0017) (end 166.9944 108.0017) (width 0.2) (layer "F.Cu") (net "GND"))
 (segment (start 162.5181 112.7281) (end 163.69 113.9) (width 0.2) (layer "F.Cu") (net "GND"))
 (segment (start 162.5181 108.7719) (end 162.5181 112.7281) (width 0.2) (layer "F.Cu") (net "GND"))
 (segment (start 143.1885 99.38) (end 152.5461 108.7376) (width 0.2) (layer "B.Cu") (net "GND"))
 (segment (start 152.5461 108.7376) (end 162.5524 108.7376) (width 0.2) (layer "B.Cu") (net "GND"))
 (segment (start 162.5524 108.7376) (end 163.69 107.6) (width 0.2) (layer "B.Cu") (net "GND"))
 (segment (start 165.6811 89.8) (end 166.7 89.8) (width 0.2) (layer "F.Cu") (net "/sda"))
 (segment (start 154.81 78.9289) (end 165.6811 89.8) (width 0.2) (layer "F.Cu") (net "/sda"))
 (segment (start 165.131 90.3501) (end 165.6811 89.8) (width 0.2) (layer "F.Cu") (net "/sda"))
 (segment (start 150.8085 114.62) (end 150.8085 115.455) (width 0.2) (layer "F.Cu") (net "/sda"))
 (segment (start 152.3765 117.023) (end 154.1264 117.023) (width 0.2) (layer "F.Cu") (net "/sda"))
 (segment (start 154.6185 116.5309) (end 154.6185 106.5215) (width 0.2) (layer "F.Cu") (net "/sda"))
 (segment (start 154.6185 106.5215) (end 161.19 99.95) (width 0.2) (layer "F.Cu") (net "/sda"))
 (segment (start 154.1264 117.023) (end 154.6185 116.5309) (width 0.2) (layer "F.Cu") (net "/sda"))
 (segment (start 161.19 99.95) (end 165.131 96.009) (width 0.2) (layer "F.Cu") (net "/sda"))
 (segment (start 154.81 70) (end 154.81 78.9289) (width 0.2) (layer "F.Cu") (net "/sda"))
 (segment (start 165.131 96.009) (end 165.131 90.3501) (width 0.2) (layer "F.Cu") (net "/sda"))
 (segment (start 150.8085 115.455) (end 152.3765 117.023) (width 0.2) (layer "F.Cu") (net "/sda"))
 (segment (start 153.3485 114.62) (end 152.27 113.5415) (width 0.2) (layer "F.Cu") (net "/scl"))
 (segment (start 155.2757 68.9363) (end 153.3337 68.9363) (width 0.2) (layer "F.Cu") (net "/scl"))
 (segment (start 152.27 113.5415) (end 152.27 70) (width 0.2) (layer "F.Cu") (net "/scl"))
 (segment (start 165.1107 78.7713) (end 155.2757 68.9363) (width 0.2) (layer "F.Cu") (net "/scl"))
 (segment (start 167.2 89.1967) (end 165.1107 87.1074) (width 0.2) (layer "F.Cu") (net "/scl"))
 (segment (start 165.1107 87.1074) (end 165.1107 78.7713) (width 0.2) (layer "F.Cu") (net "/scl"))
 (segment (start 167.2 89.8) (end 167.2 89.1967) (width 0.2) (layer "F.Cu") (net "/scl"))
 (segment (start 153.3337 68.9363) (end 152.27 70) (width 0.2) (layer "F.Cu") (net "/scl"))
 (segment (start 153.3485 114.62) (end 153.3485 115.455) (width 0.2) (layer "F.Cu") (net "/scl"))
 (segment (start 140.6485 98.545) (end 140.6485 99.38) (width 0.2) (layer "F.Cu") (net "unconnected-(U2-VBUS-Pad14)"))
 (segment (start 140.6485 114.62) (end 140.6485 115.455) (width 0.2) (layer "F.Cu") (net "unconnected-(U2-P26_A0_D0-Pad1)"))
 (segment (start 145.7285 98.545) (end 145.7285 99.38) (width 0.2) (layer "F.Cu") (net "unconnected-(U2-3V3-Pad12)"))
 (segment (start 145.7285 114.62) (end 145.7285 115.455) (width 0.2) (layer "F.Cu") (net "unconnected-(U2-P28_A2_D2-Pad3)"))
 (segment (start 150.8085 98.545) (end 150.8085 99.38) (width 0.2) (layer "F.Cu") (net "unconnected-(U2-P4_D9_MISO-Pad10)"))
 (segment (start 153.3485 98.545) (end 153.3485 99.38) (width 0.2) (layer "F.Cu") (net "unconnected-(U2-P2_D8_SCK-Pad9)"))
 (segment (start 155.8885 98.545) (end 155.8885 99.38) (width 0.2) (layer "F.Cu") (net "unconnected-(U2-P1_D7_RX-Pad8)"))
 (segment (start 148.2685 114.62) (end 148.2685 115.455) (width 0.2) (layer "F.Cu") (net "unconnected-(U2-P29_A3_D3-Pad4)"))
 (segment (start 148.2685 98.545) (end 148.2685 99.38) (width 0.2) (layer "F.Cu") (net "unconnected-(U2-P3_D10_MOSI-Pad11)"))
 (segment (start 143.1885 114.62) (end 143.1885 115.455) (width 0.2) (layer "F.Cu") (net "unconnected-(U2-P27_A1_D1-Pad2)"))
 (segment (start 171.0777 108.0746) (end 171.0777 90.5717) (width 0.2) (layer "F.Cu") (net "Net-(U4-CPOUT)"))
 (segment (start 162.299 115.009) (end 164.1433 115.009) (width 0.2) (layer "F.Cu") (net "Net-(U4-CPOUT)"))
 (segment (start 168.7 89.256) (end 168.7 89.8) (width 0.2) (layer "F.Cu") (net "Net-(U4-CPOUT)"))
 (segment (start 171.0777 90.5717) (end 169.5575 89.0515) (width 0.2) (layer "F.Cu") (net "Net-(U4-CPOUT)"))
 (segment (start 169.5575 89.0515) (end 168.9045 89.0515) (width 0.2) (layer "F.Cu") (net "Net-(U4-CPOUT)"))
 (segment (start 161.19 113.9) (end 162.299 115.009) (width 0.2) (layer "F.Cu") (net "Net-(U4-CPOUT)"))
 (segment (start 164.1433 115.009) (end 171.0777 108.0746) (width 0.2) (layer "F.Cu") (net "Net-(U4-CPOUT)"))
 (segment (start 168.9045 89.0515) (end 168.7 89.256) (width 0.2) (layer "F.Cu") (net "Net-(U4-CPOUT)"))
 (segment (start 155.8885 111.3297) (end 155.8885 114.62) (width 0.2) (layer "F.Cu") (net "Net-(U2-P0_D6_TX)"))
 (segment (start 164.6998 106.4634) (end 160.7548 106.4634) (width 0.2) (layer "F.Cu") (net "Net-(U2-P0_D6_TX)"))
 (segment (start 160.7548 106.4634) (end 155.8885 111.3297) (width 0.2) (layer "F.Cu") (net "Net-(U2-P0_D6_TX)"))
 (segment (start 170.093 94.6062) (end 170.093 104.3351) (width 0.2) (layer "F.Cu") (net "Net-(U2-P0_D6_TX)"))
 (segment (start 155.8885 114.62) (end 155.8885 115.455) (width 0.2) (layer "F.Cu") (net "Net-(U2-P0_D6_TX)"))
 (segment (start 169.2 93.7132) (end 170.093 94.6062) (width 0.2) (layer "F.Cu") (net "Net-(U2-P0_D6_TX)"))
 (segment (start 165.8364 107.6) (end 164.6998 106.4634) (width 0.2) (layer "F.Cu") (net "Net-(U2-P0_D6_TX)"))
 (segment (start 166.8281 107.6) (end 165.8364 107.6) (width 0.2) (layer "F.Cu") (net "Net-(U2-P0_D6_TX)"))
 (segment (start 170.093 104.3351) (end 166.8281 107.6) (width 0.2) (layer "F.Cu") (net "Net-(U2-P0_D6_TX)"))
 (segment (start 169.2 93.7) (end 169.2 93.7132) (width 0.2) (layer "F.Cu") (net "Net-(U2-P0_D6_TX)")))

